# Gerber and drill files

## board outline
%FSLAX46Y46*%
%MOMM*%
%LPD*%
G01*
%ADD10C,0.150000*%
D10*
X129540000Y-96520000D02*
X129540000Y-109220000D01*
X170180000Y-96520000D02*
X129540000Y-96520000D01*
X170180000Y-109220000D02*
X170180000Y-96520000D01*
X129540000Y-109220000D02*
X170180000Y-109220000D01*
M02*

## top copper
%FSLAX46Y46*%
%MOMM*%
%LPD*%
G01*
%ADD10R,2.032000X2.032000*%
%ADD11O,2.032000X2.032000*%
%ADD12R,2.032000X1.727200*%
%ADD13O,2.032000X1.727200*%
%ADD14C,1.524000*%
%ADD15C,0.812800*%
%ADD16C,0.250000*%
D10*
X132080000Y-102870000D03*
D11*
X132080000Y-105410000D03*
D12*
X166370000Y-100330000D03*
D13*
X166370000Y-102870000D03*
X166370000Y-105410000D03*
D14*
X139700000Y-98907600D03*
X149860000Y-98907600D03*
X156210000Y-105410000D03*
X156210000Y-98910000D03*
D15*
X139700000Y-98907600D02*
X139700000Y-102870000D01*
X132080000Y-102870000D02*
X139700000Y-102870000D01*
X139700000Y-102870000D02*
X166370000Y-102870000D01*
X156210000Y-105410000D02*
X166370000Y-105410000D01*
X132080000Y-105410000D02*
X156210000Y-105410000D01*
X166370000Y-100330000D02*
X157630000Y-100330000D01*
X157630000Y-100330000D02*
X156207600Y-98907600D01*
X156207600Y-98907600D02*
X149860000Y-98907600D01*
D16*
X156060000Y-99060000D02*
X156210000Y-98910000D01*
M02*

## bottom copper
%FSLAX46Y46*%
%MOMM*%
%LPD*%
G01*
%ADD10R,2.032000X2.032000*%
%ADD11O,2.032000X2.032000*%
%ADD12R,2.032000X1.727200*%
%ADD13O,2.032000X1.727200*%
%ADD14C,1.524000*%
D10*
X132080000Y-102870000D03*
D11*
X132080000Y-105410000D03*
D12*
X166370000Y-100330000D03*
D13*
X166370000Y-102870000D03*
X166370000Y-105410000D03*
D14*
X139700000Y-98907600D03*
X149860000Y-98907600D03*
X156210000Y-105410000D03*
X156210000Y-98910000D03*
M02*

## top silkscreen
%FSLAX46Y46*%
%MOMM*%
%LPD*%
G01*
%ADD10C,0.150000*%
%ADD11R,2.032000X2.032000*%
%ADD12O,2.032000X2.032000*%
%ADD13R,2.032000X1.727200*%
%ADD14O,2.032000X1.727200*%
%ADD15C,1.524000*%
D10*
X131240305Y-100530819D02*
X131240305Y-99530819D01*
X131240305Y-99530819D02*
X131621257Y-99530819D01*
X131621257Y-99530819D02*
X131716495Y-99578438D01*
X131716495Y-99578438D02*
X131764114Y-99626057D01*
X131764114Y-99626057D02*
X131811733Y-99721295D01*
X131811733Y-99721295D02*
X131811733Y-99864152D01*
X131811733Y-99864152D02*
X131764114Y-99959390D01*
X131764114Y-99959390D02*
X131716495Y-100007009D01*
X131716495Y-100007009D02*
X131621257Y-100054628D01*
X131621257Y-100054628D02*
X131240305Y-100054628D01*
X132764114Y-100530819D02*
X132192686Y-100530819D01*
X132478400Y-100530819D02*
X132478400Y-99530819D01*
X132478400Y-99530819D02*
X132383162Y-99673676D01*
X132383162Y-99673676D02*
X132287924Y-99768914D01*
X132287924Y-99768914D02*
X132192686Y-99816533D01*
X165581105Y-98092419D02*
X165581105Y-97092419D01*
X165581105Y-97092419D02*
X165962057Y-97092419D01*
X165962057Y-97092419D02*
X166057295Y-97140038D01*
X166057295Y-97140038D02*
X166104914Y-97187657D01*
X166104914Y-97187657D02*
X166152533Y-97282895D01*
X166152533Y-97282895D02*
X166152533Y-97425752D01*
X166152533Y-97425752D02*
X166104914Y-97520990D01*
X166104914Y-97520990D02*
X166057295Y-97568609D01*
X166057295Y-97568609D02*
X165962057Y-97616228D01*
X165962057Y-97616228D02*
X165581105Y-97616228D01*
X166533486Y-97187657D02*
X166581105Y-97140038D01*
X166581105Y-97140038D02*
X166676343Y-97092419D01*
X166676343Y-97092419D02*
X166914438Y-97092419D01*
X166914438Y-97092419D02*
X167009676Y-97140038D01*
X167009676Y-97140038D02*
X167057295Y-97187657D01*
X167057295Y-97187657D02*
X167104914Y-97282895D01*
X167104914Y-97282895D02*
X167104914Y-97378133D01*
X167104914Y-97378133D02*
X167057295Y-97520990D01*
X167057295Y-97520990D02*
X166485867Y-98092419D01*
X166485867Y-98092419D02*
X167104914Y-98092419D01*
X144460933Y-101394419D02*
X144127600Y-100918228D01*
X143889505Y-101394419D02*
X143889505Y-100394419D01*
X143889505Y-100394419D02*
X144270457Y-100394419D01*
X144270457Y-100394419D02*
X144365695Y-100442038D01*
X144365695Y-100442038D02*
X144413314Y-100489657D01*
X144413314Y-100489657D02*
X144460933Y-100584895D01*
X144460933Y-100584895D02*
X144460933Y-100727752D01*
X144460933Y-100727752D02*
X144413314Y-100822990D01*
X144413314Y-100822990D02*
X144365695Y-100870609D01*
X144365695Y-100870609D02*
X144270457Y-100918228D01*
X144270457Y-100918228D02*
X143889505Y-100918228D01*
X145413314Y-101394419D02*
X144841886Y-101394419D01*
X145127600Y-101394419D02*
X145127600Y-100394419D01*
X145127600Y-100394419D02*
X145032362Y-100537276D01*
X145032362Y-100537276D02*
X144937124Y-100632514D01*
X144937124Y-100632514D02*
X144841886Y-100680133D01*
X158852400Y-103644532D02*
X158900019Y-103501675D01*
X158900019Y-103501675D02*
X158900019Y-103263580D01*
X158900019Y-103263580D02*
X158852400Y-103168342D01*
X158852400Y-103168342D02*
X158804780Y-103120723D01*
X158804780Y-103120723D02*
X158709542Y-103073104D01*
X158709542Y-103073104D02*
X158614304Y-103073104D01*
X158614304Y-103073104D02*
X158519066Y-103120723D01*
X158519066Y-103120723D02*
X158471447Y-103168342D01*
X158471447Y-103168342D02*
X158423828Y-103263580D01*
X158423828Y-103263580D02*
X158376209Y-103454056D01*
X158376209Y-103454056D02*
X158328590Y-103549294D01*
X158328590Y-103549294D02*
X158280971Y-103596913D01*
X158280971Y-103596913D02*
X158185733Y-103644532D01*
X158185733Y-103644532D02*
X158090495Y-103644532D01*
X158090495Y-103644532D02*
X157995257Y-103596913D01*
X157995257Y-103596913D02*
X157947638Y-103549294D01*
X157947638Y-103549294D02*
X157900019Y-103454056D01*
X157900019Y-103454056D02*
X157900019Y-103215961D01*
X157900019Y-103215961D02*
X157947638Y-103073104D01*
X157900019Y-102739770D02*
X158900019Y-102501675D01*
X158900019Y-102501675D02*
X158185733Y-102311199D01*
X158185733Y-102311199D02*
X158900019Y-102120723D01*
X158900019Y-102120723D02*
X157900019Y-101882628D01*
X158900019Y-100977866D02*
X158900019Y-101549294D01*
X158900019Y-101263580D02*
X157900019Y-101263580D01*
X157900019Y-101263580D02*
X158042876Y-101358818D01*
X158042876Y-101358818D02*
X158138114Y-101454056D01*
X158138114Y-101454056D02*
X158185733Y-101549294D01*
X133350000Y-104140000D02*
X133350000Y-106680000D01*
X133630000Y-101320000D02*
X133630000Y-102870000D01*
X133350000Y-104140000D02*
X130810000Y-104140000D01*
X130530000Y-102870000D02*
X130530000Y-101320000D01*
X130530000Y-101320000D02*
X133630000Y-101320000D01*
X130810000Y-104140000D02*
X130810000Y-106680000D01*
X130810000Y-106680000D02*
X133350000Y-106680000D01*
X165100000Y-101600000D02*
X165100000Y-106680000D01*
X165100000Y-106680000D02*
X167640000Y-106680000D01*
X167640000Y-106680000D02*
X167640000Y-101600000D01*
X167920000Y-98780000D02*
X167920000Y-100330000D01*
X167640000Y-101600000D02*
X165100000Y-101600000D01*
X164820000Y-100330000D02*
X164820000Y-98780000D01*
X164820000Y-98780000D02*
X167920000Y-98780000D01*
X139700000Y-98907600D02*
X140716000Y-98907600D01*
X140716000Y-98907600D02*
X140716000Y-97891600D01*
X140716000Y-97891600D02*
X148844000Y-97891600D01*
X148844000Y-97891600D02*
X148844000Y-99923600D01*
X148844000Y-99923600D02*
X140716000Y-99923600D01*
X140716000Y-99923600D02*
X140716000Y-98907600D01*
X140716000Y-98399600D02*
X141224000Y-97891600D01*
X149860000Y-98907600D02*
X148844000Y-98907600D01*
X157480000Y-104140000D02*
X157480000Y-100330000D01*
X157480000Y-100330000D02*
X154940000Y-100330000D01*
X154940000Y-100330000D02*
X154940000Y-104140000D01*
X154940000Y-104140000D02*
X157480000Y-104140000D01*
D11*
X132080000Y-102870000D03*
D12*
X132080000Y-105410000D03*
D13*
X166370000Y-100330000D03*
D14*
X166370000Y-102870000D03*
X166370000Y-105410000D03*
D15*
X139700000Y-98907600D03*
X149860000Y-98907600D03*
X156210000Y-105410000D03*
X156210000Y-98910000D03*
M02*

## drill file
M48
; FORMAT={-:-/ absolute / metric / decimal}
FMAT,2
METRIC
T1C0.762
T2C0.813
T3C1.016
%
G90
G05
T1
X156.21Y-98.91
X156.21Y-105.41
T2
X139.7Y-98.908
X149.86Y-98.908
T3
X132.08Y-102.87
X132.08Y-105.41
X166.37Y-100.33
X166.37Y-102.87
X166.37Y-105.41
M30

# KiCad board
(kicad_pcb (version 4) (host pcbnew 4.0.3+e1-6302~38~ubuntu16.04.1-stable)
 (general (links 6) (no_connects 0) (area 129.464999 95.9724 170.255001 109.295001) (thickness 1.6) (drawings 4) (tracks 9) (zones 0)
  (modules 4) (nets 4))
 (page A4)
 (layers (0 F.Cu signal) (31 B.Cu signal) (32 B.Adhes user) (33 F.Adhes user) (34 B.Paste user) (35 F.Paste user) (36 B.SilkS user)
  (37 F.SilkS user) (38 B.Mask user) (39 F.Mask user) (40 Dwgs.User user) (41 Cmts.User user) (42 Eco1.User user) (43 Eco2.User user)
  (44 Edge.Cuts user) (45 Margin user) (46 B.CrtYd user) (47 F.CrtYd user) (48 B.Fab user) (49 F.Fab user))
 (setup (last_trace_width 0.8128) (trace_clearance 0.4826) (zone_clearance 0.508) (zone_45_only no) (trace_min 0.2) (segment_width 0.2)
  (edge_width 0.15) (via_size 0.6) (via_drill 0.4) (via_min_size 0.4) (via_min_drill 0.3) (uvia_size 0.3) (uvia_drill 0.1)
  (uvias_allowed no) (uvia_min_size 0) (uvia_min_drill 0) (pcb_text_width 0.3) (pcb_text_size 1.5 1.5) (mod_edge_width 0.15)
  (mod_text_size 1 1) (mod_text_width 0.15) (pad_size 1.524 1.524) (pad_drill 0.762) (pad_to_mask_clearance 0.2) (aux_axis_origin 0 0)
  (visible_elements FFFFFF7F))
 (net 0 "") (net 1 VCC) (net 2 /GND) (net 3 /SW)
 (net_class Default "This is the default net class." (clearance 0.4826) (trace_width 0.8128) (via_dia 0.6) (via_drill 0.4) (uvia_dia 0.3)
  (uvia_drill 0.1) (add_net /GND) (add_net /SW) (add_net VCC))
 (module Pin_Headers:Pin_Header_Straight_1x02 (layer F.Cu) (at 132.08 102.87)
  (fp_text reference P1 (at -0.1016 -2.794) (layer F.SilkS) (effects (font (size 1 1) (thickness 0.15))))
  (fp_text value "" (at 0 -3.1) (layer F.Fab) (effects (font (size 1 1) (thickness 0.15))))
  (fp_line (start 1.27 1.27) (end 1.27 3.81) (layer F.SilkS) (width 0.15))
  (fp_line (start 1.55 -1.55) (end 1.55 0) (layer F.SilkS) (width 0.15))
  (fp_line (start 1.27 1.27) (end -1.27 1.27) (layer F.SilkS) (width 0.15))
  (fp_line (start -1.55 0) (end -1.55 -1.55) (layer F.SilkS) (width 0.15))
  (fp_line (start -1.55 -1.55) (end 1.55 -1.55) (layer F.SilkS) (width 0.15))
  (fp_line (start -1.27 1.27) (end -1.27 3.81) (layer F.SilkS) (width 0.15))
  (fp_line (start -1.27 3.81) (end 1.27 3.81) (layer F.SilkS) (width 0.15))
  (pad 1 thru_hole rect (at 0 0) (size 2.032 2.032) (drill 1.016) (layers *.Cu *.Mask F.SilkS) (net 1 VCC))
  (pad 2 thru_hole oval (at 0 2.54) (size 2.032 2.032) (drill 1.016) (layers *.Cu *.Mask F.SilkS) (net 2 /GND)))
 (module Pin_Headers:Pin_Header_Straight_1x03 (layer F.Cu) (at 166.37 100.33)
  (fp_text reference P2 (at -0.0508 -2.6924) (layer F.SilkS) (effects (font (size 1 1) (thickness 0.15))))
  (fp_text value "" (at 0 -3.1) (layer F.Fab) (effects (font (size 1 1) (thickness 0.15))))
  (fp_line (start -1.27 1.27) (end -1.27 6.35) (layer F.SilkS) (width 0.15))
  (fp_line (start -1.27 6.35) (end 1.27 6.35) (layer F.SilkS) (width 0.15))
  (fp_line (start 1.27 6.35) (end 1.27 1.27) (layer F.SilkS) (width 0.15))
  (fp_line (start 1.55 -1.55) (end 1.55 0) (layer F.SilkS) (width 0.15))
  (fp_line (start 1.27 1.27) (end -1.27 1.27) (layer F.SilkS) (width 0.15))
  (fp_line (start -1.55 0) (end -1.55 -1.55) (layer F.SilkS) (width 0.15))
  (fp_line (start -1.55 -1.55) (end 1.55 -1.55) (layer F.SilkS) (width 0.15))
  (pad 1 thru_hole rect (at 0 0) (size 2.032 1.7272) (drill 1.016) (layers *.Cu *.Mask F.SilkS) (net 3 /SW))
  (pad 2 thru_hole oval (at 0 2.54) (size 2.032 1.7272) (drill 1.016) (layers *.Cu *.Mask F.SilkS) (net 1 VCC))
  (pad 3 thru_hole oval (at 0 5.08) (size 2.032 1.7272) (drill 1.016) (layers *.Cu *.Mask F.SilkS) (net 2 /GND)))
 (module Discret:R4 (layer F.Cu) (at 144.78 98.9076)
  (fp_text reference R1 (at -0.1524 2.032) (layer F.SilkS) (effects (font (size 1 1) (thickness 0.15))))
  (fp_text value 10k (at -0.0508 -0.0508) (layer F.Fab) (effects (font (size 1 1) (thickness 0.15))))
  (fp_line (start -5.08 0) (end -4.064 0) (layer F.SilkS) (width 0.15))
  (fp_line (start -4.064 0) (end -4.064 -1.016) (layer F.SilkS) (width 0.15))
  (fp_line (start -4.064 -1.016) (end 4.064 -1.016) (layer F.SilkS) (width 0.15))
  (fp_line (start 4.064 -1.016) (end 4.064 1.016) (layer F.SilkS) (width 0.15))
  (fp_line (start 4.064 1.016) (end -4.064 1.016) (layer F.SilkS) (width 0.15))
  (fp_line (start -4.064 1.016) (end -4.064 0) (layer F.SilkS) (width 0.15))
  (fp_line (start -4.064 -0.508) (end -3.556 -1.016) (layer F.SilkS) (width 0.15))
  (fp_line (start 5.08 0) (end 4.064 0) (layer F.SilkS) (width 0.15))
  (pad 1 thru_hole circle (at -5.08 0) (size 1.524 1.524) (drill 0.8128) (layers *.Cu *.Mask F.SilkS) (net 1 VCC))
  (pad 2 thru_hole circle (at 5.08 0) (size 1.524 1.524) (drill 0.8128) (layers *.Cu *.Mask F.SilkS) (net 3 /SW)))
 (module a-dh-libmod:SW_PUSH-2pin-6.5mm (layer F.Cu) (at 153.67 105.41 90)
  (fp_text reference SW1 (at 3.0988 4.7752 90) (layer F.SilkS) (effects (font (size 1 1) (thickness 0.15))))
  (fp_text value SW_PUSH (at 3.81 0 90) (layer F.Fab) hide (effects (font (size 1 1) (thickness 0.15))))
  (fp_line (start 1.27 3.81) (end 5.08 3.81) (layer F.SilkS) (width 0.15))
  (fp_line (start 5.08 3.81) (end 5.08 1.27) (layer F.SilkS) (width 0.15))
  (fp_line (start 5.08 1.27) (end 1.27 1.27) (layer F.SilkS) (width 0.15))
  (fp_line (start 1.27 1.27) (end 1.27 3.81) (layer F.SilkS) (width 0.15))
  (pad 1 thru_hole circle (at 0 2.54 90) (size 1.524 1.524) (drill 0.762) (layers *.Cu *.Mask F.SilkS) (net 2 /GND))
  (pad 2 thru_hole circle (at 6.5 2.54 90) (size 1.524 1.524) (drill 0.762) (layers *.Cu *.Mask F.SilkS) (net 3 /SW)))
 (gr_line (start 129.54 96.52) (end 129.54 109.22) (angle 90) (layer Edge.Cuts) (width 0.15))
 (gr_line (start 170.18 96.52) (end 129.54 96.52) (angle 90) (layer Edge.Cuts) (width 0.15))
 (gr_line (start 170.18 109.22) (end 170.18 96.52) (angle 90) (layer Edge.Cuts) (width 0.15))
 (gr_line (start 129.54 109.22) (end 170.18 109.22) (angle 90) (layer Edge.Cuts) (width 0.15))
 (segment (start 139.7 98.9076) (end 139.7 102.87) (width 0.8128) (layer F.Cu) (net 1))
 (segment (start 132.08 102.87) (end 139.7 102.87) (width 0.8128) (layer F.Cu) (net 1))
 (segment (start 139.7 102.87) (end 166.37 102.87) (width 0.8128) (layer F.Cu) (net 1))
 (segment (start 156.21 105.41) (end 166.37 105.41) (width 0.8128) (layer F.Cu) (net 2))
 (segment (start 132.08 105.41) (end 156.21 105.41) (width 0.8128) (layer F.Cu) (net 2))
 (segment (start 166.37 100.33) (end 157.63 100.33) (width 0.8128) (layer F.Cu) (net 3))
 (segment (start 157.63 100.33) (end 156.2076 98.9076) (width 0.8128) (layer F.Cu) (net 3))
 (segment (start 156.2076 98.9076) (end 149.86 98.9076) (width 0.8128) (layer F.Cu) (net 3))
 (segment (start 156.06 99.06) (end 156.21 98.91) (width 0.25) (layer F.Cu) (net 3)))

